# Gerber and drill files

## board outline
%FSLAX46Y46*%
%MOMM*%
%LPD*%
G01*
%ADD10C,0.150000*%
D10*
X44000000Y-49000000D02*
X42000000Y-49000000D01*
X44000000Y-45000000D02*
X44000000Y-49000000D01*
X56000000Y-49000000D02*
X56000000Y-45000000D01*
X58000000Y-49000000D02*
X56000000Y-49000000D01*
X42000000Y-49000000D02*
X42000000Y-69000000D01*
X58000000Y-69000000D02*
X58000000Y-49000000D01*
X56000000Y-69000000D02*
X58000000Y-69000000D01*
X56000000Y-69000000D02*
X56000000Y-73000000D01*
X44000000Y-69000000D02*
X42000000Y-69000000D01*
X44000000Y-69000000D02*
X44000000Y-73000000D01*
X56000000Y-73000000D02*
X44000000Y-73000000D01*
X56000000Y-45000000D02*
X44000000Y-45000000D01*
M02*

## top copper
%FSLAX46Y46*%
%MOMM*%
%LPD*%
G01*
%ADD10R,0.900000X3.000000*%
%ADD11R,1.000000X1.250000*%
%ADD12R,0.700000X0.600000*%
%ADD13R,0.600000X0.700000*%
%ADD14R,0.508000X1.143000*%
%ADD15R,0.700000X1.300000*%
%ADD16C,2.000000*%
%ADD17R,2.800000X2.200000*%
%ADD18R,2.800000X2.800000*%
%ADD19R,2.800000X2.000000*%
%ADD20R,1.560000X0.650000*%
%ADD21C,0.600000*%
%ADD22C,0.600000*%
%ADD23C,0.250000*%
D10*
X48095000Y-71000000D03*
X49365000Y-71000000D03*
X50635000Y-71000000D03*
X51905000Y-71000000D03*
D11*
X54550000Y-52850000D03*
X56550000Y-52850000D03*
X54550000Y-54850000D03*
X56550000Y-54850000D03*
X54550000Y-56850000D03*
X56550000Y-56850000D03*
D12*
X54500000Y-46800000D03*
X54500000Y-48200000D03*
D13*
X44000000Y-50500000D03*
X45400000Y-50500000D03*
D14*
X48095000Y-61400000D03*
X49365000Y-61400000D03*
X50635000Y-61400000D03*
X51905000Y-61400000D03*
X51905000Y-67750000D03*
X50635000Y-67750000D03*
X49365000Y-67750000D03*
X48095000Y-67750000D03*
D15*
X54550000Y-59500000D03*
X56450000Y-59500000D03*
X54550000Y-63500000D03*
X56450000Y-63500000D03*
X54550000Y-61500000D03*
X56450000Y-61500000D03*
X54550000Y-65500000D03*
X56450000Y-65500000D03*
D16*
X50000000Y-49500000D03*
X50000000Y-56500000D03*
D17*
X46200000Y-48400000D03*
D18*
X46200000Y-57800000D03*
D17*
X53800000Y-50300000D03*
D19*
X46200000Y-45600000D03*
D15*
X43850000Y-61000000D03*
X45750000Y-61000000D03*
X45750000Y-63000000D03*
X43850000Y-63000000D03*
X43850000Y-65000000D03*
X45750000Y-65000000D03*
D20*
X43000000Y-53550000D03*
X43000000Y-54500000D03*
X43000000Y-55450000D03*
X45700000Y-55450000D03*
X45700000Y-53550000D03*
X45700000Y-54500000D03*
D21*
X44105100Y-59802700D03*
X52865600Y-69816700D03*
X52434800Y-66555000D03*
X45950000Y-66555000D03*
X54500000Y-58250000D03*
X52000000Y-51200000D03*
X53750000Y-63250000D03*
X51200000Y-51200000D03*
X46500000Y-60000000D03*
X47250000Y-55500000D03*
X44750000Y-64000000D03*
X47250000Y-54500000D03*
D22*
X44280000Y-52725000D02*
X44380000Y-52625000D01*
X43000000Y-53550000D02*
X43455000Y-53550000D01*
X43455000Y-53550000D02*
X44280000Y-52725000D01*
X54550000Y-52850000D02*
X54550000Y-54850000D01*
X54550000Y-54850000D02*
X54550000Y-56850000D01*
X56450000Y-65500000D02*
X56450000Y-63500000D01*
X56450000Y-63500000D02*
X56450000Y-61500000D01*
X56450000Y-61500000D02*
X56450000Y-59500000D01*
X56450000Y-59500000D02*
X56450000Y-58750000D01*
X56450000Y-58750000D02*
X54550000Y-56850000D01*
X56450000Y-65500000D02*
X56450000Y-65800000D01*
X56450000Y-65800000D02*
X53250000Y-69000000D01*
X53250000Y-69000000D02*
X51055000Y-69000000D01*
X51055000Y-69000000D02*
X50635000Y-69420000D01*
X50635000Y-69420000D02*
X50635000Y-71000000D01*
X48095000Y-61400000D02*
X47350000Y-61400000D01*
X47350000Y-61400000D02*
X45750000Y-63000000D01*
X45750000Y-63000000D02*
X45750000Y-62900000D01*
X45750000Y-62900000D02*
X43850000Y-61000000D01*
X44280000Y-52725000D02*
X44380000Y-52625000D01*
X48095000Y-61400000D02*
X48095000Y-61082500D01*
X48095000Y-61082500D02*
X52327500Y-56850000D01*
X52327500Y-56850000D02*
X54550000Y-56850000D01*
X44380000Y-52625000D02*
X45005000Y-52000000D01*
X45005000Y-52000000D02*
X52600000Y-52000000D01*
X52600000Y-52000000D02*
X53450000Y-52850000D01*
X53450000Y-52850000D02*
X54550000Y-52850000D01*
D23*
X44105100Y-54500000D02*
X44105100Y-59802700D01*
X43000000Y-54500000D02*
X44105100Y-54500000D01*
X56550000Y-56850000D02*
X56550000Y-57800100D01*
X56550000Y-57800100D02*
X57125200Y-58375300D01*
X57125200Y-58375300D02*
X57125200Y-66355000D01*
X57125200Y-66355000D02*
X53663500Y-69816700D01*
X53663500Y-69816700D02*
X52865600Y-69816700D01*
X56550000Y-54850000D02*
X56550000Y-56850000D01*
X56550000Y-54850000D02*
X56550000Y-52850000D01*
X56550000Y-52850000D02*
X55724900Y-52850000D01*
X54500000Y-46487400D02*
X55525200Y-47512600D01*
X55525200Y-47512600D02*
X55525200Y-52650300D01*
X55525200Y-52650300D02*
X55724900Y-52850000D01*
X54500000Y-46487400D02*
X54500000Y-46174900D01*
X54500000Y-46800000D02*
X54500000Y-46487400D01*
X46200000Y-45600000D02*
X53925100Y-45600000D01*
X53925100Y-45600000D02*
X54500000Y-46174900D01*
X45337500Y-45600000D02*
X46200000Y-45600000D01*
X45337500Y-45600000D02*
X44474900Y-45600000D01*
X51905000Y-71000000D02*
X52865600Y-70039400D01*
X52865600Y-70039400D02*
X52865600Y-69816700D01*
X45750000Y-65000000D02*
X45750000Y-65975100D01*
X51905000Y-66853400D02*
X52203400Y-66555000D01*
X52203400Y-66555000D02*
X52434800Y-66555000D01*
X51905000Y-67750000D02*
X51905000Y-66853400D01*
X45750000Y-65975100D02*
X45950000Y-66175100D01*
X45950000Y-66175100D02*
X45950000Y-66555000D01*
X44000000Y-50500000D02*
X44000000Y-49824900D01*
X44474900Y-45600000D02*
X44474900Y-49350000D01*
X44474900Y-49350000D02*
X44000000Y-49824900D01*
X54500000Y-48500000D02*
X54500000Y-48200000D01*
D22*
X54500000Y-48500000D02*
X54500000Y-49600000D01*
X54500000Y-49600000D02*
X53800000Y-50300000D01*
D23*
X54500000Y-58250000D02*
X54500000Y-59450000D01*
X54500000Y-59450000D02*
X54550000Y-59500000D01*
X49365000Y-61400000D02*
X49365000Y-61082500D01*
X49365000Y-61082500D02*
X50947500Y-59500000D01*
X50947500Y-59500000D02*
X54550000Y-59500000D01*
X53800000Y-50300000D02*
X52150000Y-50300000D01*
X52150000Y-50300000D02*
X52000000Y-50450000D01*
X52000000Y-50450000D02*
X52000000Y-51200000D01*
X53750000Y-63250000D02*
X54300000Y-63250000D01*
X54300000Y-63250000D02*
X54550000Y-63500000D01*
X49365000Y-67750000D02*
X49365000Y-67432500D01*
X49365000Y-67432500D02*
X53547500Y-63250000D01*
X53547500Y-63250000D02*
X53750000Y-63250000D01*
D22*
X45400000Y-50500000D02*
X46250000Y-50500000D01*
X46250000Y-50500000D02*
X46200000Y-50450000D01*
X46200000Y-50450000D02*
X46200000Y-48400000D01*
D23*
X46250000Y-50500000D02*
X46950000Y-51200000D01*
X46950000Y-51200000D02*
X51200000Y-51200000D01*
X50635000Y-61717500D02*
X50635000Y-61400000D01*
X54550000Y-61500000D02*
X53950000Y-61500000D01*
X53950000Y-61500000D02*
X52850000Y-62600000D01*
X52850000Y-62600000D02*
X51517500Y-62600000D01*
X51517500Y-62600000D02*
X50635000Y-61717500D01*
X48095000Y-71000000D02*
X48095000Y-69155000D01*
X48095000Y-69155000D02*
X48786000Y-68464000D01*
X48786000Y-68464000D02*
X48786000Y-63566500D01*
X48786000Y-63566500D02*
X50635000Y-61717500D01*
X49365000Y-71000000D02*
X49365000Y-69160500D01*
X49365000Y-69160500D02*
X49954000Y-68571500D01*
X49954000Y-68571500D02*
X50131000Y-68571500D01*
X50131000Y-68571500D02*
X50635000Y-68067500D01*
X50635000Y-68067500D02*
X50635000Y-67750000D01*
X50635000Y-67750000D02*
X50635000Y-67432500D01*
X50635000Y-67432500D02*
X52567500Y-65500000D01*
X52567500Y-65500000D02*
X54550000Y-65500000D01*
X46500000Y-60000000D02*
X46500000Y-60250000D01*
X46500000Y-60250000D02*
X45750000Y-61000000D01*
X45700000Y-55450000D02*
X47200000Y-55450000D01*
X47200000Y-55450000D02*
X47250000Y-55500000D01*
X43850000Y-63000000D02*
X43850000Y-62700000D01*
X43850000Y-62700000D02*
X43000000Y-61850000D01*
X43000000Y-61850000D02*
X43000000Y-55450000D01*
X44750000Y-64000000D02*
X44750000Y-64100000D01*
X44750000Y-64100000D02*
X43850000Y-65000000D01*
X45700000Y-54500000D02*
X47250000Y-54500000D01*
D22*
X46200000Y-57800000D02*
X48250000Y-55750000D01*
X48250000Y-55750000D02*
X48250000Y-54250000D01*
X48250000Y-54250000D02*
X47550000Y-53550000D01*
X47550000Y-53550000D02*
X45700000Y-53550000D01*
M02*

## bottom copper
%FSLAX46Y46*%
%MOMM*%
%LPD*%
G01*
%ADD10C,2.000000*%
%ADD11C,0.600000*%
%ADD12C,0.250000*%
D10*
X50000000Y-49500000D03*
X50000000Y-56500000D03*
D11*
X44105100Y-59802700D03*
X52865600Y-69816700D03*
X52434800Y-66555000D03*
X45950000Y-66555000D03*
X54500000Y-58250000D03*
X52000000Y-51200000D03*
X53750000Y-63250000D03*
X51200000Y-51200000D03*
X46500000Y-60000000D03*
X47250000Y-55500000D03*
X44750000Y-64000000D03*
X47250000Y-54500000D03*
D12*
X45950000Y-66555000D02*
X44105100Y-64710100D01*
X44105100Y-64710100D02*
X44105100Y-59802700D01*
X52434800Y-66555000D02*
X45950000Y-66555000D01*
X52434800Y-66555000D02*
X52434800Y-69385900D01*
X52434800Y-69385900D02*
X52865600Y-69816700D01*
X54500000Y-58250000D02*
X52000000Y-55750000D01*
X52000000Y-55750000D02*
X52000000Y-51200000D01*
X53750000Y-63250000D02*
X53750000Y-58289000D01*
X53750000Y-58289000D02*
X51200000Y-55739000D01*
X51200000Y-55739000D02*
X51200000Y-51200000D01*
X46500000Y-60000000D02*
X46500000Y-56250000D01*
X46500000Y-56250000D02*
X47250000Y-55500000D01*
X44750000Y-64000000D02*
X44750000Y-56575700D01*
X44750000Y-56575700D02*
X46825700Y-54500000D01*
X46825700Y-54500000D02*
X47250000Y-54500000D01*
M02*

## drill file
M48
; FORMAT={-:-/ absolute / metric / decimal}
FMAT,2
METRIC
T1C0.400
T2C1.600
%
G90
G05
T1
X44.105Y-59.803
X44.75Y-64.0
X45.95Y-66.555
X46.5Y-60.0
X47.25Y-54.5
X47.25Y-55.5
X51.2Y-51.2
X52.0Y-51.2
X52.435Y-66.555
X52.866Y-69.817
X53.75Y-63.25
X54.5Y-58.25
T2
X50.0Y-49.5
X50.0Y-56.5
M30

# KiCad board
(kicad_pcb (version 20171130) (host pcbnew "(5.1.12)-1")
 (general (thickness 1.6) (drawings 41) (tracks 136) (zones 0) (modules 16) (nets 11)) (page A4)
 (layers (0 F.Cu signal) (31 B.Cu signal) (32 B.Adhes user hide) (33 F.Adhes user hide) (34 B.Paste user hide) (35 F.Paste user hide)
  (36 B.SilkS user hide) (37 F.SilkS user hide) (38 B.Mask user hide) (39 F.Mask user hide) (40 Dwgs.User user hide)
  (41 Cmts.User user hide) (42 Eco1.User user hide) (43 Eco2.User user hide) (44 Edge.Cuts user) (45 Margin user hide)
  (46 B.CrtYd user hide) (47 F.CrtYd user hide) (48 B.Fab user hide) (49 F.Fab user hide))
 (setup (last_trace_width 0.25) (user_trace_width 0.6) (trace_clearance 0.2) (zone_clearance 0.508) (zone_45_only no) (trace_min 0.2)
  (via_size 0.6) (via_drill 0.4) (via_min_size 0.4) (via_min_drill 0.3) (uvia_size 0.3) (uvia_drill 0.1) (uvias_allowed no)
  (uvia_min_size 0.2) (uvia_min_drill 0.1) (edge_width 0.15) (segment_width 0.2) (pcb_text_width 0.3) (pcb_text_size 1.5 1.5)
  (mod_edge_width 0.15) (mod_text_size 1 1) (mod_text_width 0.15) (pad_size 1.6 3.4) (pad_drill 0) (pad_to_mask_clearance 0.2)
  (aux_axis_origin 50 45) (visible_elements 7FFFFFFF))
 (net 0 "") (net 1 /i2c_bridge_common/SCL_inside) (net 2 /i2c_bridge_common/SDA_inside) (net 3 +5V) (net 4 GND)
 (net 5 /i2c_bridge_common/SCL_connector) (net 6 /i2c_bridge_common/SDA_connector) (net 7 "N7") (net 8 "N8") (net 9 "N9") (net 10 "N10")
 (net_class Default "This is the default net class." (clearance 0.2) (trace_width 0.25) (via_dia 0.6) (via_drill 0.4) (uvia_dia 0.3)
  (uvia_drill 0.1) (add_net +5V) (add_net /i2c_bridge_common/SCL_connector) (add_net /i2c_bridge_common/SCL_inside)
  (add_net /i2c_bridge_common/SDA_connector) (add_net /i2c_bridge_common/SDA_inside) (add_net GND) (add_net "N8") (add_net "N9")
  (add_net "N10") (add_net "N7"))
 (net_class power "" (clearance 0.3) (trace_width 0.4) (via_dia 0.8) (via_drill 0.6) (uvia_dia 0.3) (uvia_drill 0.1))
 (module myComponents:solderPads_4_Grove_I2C (layer F.Cu) (at 50 71)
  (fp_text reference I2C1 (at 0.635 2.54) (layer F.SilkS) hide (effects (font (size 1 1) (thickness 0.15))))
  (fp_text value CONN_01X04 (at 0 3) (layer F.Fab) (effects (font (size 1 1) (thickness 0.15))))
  (pad 1 smd rect (at -1.905 0) (size 0.9 3) (layers F.Cu F.Paste F.Mask) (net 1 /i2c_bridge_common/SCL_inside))
  (pad 2 smd rect (at -0.635 0) (size 0.9 3) (layers F.Cu F.Paste F.Mask) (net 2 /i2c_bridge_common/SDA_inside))
  (pad 3 smd rect (at 0.635 0) (size 0.9 3) (layers F.Cu F.Paste F.Mask) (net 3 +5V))
  (pad 4 smd rect (at 1.905 0) (size 0.9 3) (layers F.Cu F.Paste F.Mask) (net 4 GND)))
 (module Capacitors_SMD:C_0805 (layer F.Cu) (at 55.55 52.85)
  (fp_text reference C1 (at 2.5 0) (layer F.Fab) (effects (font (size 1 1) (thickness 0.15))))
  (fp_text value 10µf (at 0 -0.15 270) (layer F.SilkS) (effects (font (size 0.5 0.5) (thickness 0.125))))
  (pad 1 smd rect (at -1 0) (size 1 1.25) (layers F.Cu F.Paste F.Mask) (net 3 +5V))
  (pad 2 smd rect (at 1 0) (size 1 1.25) (layers F.Cu F.Paste F.Mask) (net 4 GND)))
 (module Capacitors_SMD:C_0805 (layer F.Cu) (at 55.55 54.85)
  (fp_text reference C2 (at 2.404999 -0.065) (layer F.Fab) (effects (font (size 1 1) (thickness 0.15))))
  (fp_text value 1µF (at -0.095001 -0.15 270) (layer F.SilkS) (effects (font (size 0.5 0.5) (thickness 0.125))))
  (pad 1 smd rect (at -1 0) (size 1 1.25) (layers F.Cu F.Paste F.Mask) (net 3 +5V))
  (pad 2 smd rect (at 1 0) (size 1 1.25) (layers F.Cu F.Paste F.Mask) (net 4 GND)))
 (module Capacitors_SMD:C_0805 (layer F.Cu) (at 55.55 56.85)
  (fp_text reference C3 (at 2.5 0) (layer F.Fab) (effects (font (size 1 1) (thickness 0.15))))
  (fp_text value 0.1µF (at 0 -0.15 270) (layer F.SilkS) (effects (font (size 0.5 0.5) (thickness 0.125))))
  (pad 1 smd rect (at -1 0) (size 1 1.25) (layers F.Cu F.Paste F.Mask) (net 3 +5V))
  (pad 2 smd rect (at 1 0) (size 1 1.25) (layers F.Cu F.Paste F.Mask) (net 4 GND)))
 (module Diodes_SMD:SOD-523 (layer F.Cu) (at 54.5 47.5 90)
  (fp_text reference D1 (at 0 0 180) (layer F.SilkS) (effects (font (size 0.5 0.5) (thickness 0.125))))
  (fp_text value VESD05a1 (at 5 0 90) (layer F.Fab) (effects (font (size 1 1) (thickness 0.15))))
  (pad 2 smd rect (at 0.7 0 270) (size 0.6 0.7) (layers F.Cu F.Paste F.Mask) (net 4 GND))
  (pad 1 smd rect (at -0.7 0 270) (size 0.6 0.7) (layers F.Cu F.Paste F.Mask) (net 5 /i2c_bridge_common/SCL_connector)))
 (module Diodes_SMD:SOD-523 (layer F.Cu) (at 44.7 50.5 180)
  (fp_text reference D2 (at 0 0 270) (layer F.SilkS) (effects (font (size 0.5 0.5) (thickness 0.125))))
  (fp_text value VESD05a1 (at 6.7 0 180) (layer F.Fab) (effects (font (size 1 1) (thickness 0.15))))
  (pad 2 smd rect (at 0.7 0) (size 0.6 0.7) (layers F.Cu F.Paste F.Mask) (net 4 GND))
  (pad 1 smd rect (at -0.7 0) (size 0.6 0.7) (layers F.Cu F.Paste F.Mask) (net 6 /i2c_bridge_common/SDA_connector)))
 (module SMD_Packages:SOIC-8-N (layer F.Cu) (at 50 64.575)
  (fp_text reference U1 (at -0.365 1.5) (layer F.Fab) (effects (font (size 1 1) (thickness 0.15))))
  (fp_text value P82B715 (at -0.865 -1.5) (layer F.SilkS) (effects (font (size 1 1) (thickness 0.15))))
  (pad 8 smd rect (at -1.905 -3.175) (size 0.508 1.143) (layers F.Cu F.Paste F.Mask) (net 3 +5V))
  (pad 7 smd rect (at -0.635 -3.175) (size 0.508 1.143) (layers F.Cu F.Paste F.Mask) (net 5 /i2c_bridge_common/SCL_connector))
  (pad 6 smd rect (at 0.635 -3.175) (size 0.508 1.143) (layers F.Cu F.Paste F.Mask) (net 1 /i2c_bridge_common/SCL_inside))
  (pad 5 smd rect (at 1.905 -3.175) (size 0.508 1.143) (layers F.Cu F.Paste F.Mask))
  (pad 4 smd rect (at 1.905 3.175) (size 0.508 1.143) (layers F.Cu F.Paste F.Mask) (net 4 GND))
  (pad 3 smd rect (at 0.635 3.175) (size 0.508 1.143) (layers F.Cu F.Paste F.Mask) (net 2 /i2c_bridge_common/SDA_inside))
  (pad 2 smd rect (at -0.635 3.175) (size 0.508 1.143) (layers F.Cu F.Paste F.Mask) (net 6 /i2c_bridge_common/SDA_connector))
  (pad 1 smd rect (at -1.905 3.175) (size 0.508 1.143) (layers F.Cu F.Paste F.Mask)))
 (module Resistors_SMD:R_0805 (layer F.Cu) (at 55.5 59.5)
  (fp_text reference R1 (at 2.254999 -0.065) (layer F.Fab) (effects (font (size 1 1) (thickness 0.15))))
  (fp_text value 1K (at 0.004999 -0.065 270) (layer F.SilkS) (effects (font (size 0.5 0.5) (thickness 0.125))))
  (pad 1 smd rect (at -0.95 0) (size 0.7 1.3) (layers F.Cu F.Paste F.Mask) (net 5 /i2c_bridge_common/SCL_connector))
  (pad 2 smd rect (at 0.95 0) (size 0.7 1.3) (layers F.Cu F.Paste F.Mask) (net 3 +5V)))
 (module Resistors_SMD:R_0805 (layer F.Cu) (at 55.5 63.5)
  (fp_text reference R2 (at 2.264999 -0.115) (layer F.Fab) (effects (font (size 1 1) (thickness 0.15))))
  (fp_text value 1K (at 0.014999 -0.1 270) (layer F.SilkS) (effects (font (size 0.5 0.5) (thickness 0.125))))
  (pad 1 smd rect (at -0.95 0) (size 0.7 1.3) (layers F.Cu F.Paste F.Mask) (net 6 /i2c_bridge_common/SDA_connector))
  (pad 2 smd rect (at 0.95 0) (size 0.7 1.3) (layers F.Cu F.Paste F.Mask) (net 3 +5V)))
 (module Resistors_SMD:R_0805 (layer F.Cu) (at 55.5 61.5)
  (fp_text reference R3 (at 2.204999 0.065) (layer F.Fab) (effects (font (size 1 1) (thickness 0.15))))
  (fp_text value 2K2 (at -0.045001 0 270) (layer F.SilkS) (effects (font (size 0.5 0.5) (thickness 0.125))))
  (pad 1 smd rect (at -0.95 0) (size 0.7 1.3) (layers F.Cu F.Paste F.Mask) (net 1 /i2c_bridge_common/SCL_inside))
  (pad 2 smd rect (at 0.95 0) (size 0.7 1.3) (layers F.Cu F.Paste F.Mask) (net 3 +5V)))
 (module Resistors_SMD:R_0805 (layer F.Cu) (at 55.5 65.5)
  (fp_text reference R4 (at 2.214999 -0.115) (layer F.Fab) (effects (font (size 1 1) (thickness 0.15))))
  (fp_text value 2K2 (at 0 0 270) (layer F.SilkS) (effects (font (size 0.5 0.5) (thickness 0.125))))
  (pad 1 smd rect (at -0.95 0) (size 0.7 1.3) (layers F.Cu F.Paste F.Mask) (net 2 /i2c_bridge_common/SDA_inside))
  (pad 2 smd rect (at 0.95 0) (size 0.7 1.3) (layers F.Cu F.Paste F.Mask) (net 3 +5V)))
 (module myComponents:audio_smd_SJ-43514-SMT (layer F.Cu) (at 50 45 270)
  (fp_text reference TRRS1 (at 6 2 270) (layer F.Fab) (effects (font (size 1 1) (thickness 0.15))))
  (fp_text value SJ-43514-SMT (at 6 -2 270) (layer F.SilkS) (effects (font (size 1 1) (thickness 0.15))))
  (pad "" thru_hole circle (at 4.5 0 270) (size 2 2) (drill 1.6) (layers *.Cu *.Mask F.SilkS))
  (pad "" thru_hole circle (at 11.5 0 270) (size 2 2) (drill 1.6) (layers *.Cu *.Mask F.SilkS))
  (pad 4 smd rect (at 3.4 3.8 270) (size 2.2 2.8) (layers F.Cu F.Paste F.Mask) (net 6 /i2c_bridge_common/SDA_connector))
  (pad 2 smd rect (at 12.8 3.8 270) (size 2.8 2.8) (layers F.Cu F.Paste F.Mask) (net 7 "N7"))
  (pad 3 smd rect (at 5.3 -3.8 270) (size 2.2 2.8) (layers F.Cu F.Paste F.Mask) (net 5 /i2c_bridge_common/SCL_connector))
  (pad 1 smd rect (at 0.6 3.8 270) (size 2 2.8) (layers F.Cu F.Paste F.Mask) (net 4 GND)))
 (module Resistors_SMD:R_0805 (layer F.Cu) (at 44.8 61)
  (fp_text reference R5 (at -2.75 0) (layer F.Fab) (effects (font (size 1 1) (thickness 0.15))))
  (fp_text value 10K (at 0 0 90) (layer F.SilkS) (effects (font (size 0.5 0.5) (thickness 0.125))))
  (pad 1 smd rect (at -0.95 0) (size 0.7 1.3) (layers F.Cu F.Paste F.Mask) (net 3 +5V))
  (pad 2 smd rect (at 0.95 0) (size 0.7 1.3) (layers F.Cu F.Paste F.Mask) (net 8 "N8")))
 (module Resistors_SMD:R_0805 (layer F.Cu) (at 44.8 63 180)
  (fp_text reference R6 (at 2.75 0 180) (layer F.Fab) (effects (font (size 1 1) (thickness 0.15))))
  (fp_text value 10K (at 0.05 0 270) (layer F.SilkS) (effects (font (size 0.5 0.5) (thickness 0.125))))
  (pad 1 smd rect (at -0.95 0 180) (size 0.7 1.3) (layers F.Cu F.Paste F.Mask) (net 3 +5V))
  (pad 2 smd rect (at 0.95 0 180) (size 0.7 1.3) (layers F.Cu F.Paste F.Mask) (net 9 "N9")))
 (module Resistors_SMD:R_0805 (layer F.Cu) (at 44.8 65)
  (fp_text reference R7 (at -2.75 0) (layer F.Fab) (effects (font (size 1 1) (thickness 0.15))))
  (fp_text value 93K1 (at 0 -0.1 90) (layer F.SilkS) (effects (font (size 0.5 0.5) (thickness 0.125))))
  (pad 1 smd rect (at -0.95 0) (size 0.7 1.3) (layers F.Cu F.Paste F.Mask) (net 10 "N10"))
  (pad 2 smd rect (at 0.95 0) (size 0.7 1.3) (layers F.Cu F.Paste F.Mask) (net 4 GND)))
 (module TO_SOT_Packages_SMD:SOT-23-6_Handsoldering (layer F.Cu) (at 44.35 54.5)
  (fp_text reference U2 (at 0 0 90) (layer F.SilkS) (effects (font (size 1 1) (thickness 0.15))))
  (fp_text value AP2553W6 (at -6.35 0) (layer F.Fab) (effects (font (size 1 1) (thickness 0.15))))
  (pad 1 smd rect (at -1.35 -0.95) (size 1.56 0.65) (layers F.Cu F.Paste F.Mask) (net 3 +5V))
  (pad 2 smd rect (at -1.35 0) (size 1.56 0.65) (layers F.Cu F.Paste F.Mask) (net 4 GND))
  (pad 3 smd rect (at -1.35 0.95) (size 1.56 0.65) (layers F.Cu F.Paste F.Mask) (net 9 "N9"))
  (pad 4 smd rect (at 1.35 0.95) (size 1.56 0.65) (layers F.Cu F.Paste F.Mask) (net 8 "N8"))
  (pad 6 smd rect (at 1.35 -0.95) (size 1.56 0.65) (layers F.Cu F.Paste F.Mask) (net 7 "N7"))
  (pad 5 smd rect (at 1.35 0) (size 1.56 0.65) (layers F.Cu F.Paste F.Mask) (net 10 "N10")))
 (gr_line (start 44 49) (end 42 49) (layer Edge.Cuts) (width 0.15))
 (gr_line (start 44 45) (end 44 49) (layer Edge.Cuts) (width 0.15))
 (gr_line (start 56 49) (end 56 45) (layer Edge.Cuts) (width 0.15))
 (gr_line (start 58 49) (end 56 49) (layer Edge.Cuts) (width 0.15))
 (gr_line (start 42 49) (end 42 69) (layer Edge.Cuts) (width 0.15))
 (gr_line (start 58 69) (end 58 49) (layer Edge.Cuts) (width 0.15))
 (gr_line (start 56 69) (end 58 69) (layer Edge.Cuts) (width 0.15))
 (gr_line (start 56 69) (end 56 73) (layer Edge.Cuts) (width 0.15))
 (gr_line (start 44 69) (end 42 69) (layer Edge.Cuts) (width 0.15))
 (gr_line (start 44 69) (end 44 73) (layer Edge.Cuts) (width 0.15))
 (gr_line (start 56 73) (end 44 73) (layer Edge.Cuts) (width 0.15))
 (gr_line (start 56 45) (end 44 45) (layer Edge.Cuts) (width 0.15))
 (segment (start 44.28 52.725) (end 44.38 52.625) (width 0.6) (layer F.Cu) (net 3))
 (segment (start 43 53.55) (end 43.455 53.55) (width 0.6) (layer F.Cu) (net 3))
 (segment (start 43.455 53.55) (end 44.28 52.725) (width 0.6) (layer F.Cu) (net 3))
 (segment (start 54.55 52.85) (end 54.55 54.85) (width 0.6) (layer F.Cu) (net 3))
 (segment (start 54.55 54.85) (end 54.55 56.85) (width 0.6) (layer F.Cu) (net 3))
 (segment (start 56.45 65.5) (end 56.45 63.5) (width 0.6) (layer F.Cu) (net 3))
 (segment (start 56.45 63.5) (end 56.45 61.5) (width 0.6) (layer F.Cu) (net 3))
 (segment (start 56.45 61.5) (end 56.45 59.5) (width 0.6) (layer F.Cu) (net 3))
 (segment (start 56.45 59.5) (end 56.45 58.75) (width 0.6) (layer F.Cu) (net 3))
 (segment (start 56.45 58.75) (end 54.55 56.85) (width 0.6) (layer F.Cu) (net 3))
 (segment (start 56.45 65.5) (end 56.45 65.8) (width 0.6) (layer F.Cu) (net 3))
 (segment (start 56.45 65.8) (end 53.25 69) (width 0.6) (layer F.Cu) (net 3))
 (segment (start 53.25 69) (end 51.055 69) (width 0.6) (layer F.Cu) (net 3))
 (segment (start 51.055 69) (end 50.635 69.42) (width 0.6) (layer F.Cu) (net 3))
 (segment (start 50.635 69.42) (end 50.635 71) (width 0.6) (layer F.Cu) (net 3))
 (segment (start 48.095 61.4) (end 47.35 61.4) (width 0.6) (layer F.Cu) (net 3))
 (segment (start 47.35 61.4) (end 45.75 63) (width 0.6) (layer F.Cu) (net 3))
 (segment (start 45.75 63) (end 45.75 62.9) (width 0.6) (layer F.Cu) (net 3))
 (segment (start 45.75 62.9) (end 43.85 61) (width 0.6) (layer F.Cu) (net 3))
 (segment (start 44.28 52.725) (end 44.38 52.625) (width 0.6) (layer F.Cu) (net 3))
 (segment (start 48.095 61.4) (end 48.095 61.0825) (width 0.6) (layer F.Cu) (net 3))
 (segment (start 48.095 61.0825) (end 52.3275 56.85) (width 0.6) (layer F.Cu) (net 3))
 (segment (start 52.3275 56.85) (end 54.55 56.85) (width 0.6) (layer F.Cu) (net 3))
 (segment (start 44.38 52.625) (end 45.005 52) (width 0.6) (layer F.Cu) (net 3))
 (segment (start 45.005 52) (end 52.6 52) (width 0.6) (layer F.Cu) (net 3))
 (segment (start 52.6 52) (end 53.45 52.85) (width 0.6) (layer F.Cu) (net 3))
 (segment (start 53.45 52.85) (end 54.55 52.85) (width 0.6) (layer F.Cu) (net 3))
 (segment (start 44.1051 54.5) (end 44.1051 59.8027) (width 0.25) (layer F.Cu) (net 4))
 (segment (start 45.95 66.555) (end 44.1051 64.7101) (width 0.25) (layer B.Cu) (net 4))
 (segment (start 44.1051 64.7101) (end 44.1051 59.8027) (width 0.25) (layer B.Cu) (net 4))
 (segment (start 43 54.5) (end 44.1051 54.5) (width 0.25) (layer F.Cu) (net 4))
 (segment (start 52.4348 66.555) (end 45.95 66.555) (width 0.25) (layer B.Cu) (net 4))
 (segment (start 56.55 56.85) (end 56.55 57.8001) (width 0.25) (layer F.Cu) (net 4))
 (segment (start 56.55 57.8001) (end 57.1252 58.3753) (width 0.25) (layer F.Cu) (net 4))
 (segment (start 57.1252 58.3753) (end 57.1252 66.355) (width 0.25) (layer F.Cu) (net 4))
 (segment (start 57.1252 66.355) (end 53.6635 69.8167) (width 0.25) (layer F.Cu) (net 4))
 (segment (start 53.6635 69.8167) (end 52.8656 69.8167) (width 0.25) (layer F.Cu) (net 4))
 (segment (start 56.55 54.85) (end 56.55 56.85) (width 0.25) (layer F.Cu) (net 4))
 (segment (start 56.55 54.85) (end 56.55 52.85) (width 0.25) (layer F.Cu) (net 4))
 (segment (start 56.55 52.85) (end 55.7249 52.85) (width 0.25) (layer F.Cu) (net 4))
 (segment (start 54.5 46.4874) (end 55.5252 47.5126) (width 0.25) (layer F.Cu) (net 4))
 (segment (start 55.5252 47.5126) (end 55.5252 52.6503) (width 0.25) (layer F.Cu) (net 4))
 (segment (start 55.5252 52.6503) (end 55.7249 52.85) (width 0.25) (layer F.Cu) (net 4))
 (segment (start 54.5 46.4874) (end 54.5 46.1749) (width 0.25) (layer F.Cu) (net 4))
 (segment (start 54.5 46.8) (end 54.5 46.4874) (width 0.25) (layer F.Cu) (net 4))
 (segment (start 46.2 45.6) (end 53.9251 45.6) (width 0.25) (layer F.Cu) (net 4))
 (segment (start 53.9251 45.6) (end 54.5 46.1749) (width 0.25) (layer F.Cu) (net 4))
 (segment (start 45.3375 45.6) (end 46.2 45.6) (width 0.25) (layer F.Cu) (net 4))
 (segment (start 45.3375 45.6) (end 44.4749 45.6) (width 0.25) (layer F.Cu) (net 4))
 (segment (start 52.4348 66.555) (end 52.4348 69.3859) (width 0.25) (layer B.Cu) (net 4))
 (segment (start 52.4348 69.3859) (end 52.8656 69.8167) (width 0.25) (layer B.Cu) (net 4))
 (segment (start 51.905 71) (end 52.8656 70.0394) (width 0.25) (layer F.Cu) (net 4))
 (segment (start 52.8656 70.0394) (end 52.8656 69.8167) (width 0.25) (layer F.Cu) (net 4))
 (segment (start 45.75 65) (end 45.75 65.9751) (width 0.25) (layer F.Cu) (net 4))
 (segment (start 51.905 66.8534) (end 52.2034 66.555) (width 0.25) (layer F.Cu) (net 4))
 (segment (start 52.2034 66.555) (end 52.4348 66.555) (width 0.25) (layer F.Cu) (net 4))
 (segment (start 51.905 67.75) (end 51.905 66.8534) (width 0.25) (layer F.Cu) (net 4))
 (segment (start 45.75 65.9751) (end 45.95 66.1751) (width 0.25) (layer F.Cu) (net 4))
 (segment (start 45.95 66.1751) (end 45.95 66.555) (width 0.25) (layer F.Cu) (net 4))
 (segment (start 44 50.5) (end 44 49.8249) (width 0.25) (layer F.Cu) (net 4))
 (segment (start 44.4749 45.6) (end 44.4749 49.35) (width 0.25) (layer F.Cu) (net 4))
 (segment (start 44.4749 49.35) (end 44 49.8249) (width 0.25) (layer F.Cu) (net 4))
 (via (at 44.1051 59.8027) (size 0.6) (layers F.Cu B.Cu) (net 4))
 (via (at 52.8656 69.8167) (size 0.6) (layers F.Cu B.Cu) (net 4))
 (via (at 52.4348 66.555) (size 0.6) (layers F.Cu B.Cu) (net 4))
 (via (at 45.95 66.555) (size 0.6) (layers F.Cu B.Cu) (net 4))
 (segment (start 54.5 48.5) (end 54.5 48.2) (width 0.25) (layer F.Cu) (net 5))
 (segment (start 54.5 48.5) (end 54.5 49.6) (width 0.6) (layer F.Cu) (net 5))
 (segment (start 54.5 49.6) (end 53.8 50.3) (width 0.6) (layer F.Cu) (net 5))
 (segment (start 54.5 58.25) (end 54.5 59.45) (width 0.25) (layer F.Cu) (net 5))
 (segment (start 54.5 59.45) (end 54.55 59.5) (width 0.25) (layer F.Cu) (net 5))
 (segment (start 49.365 61.4) (end 49.365 61.0825) (width 0.25) (layer F.Cu) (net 5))
 (segment (start 49.365 61.0825) (end 50.9475 59.5) (width 0.25) (layer F.Cu) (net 5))
 (segment (start 50.9475 59.5) (end 54.55 59.5) (width 0.25) (layer F.Cu) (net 5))
 (segment (start 53.8 50.3) (end 52.15 50.3) (width 0.25) (layer F.Cu) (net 5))
 (segment (start 52.15 50.3) (end 52 50.45) (width 0.25) (layer F.Cu) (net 5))
 (segment (start 52 50.45) (end 52 51.2) (width 0.25) (layer F.Cu) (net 5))
 (segment (start 54.5 58.25) (end 52 55.75) (width 0.25) (layer B.Cu) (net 5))
 (segment (start 52 55.75) (end 52 51.2) (width 0.25) (layer B.Cu) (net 5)) (via (at 54.5 58.25) (size 0.6) (layers F.Cu B.Cu) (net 5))
 (via (at 52 51.2) (size 0.6) (layers F.Cu B.Cu) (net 5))
 (segment (start 53.75 63.25) (end 54.3 63.25) (width 0.25) (layer F.Cu) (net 6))
 (segment (start 54.3 63.25) (end 54.55 63.5) (width 0.25) (layer F.Cu) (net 6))
 (segment (start 49.365 67.75) (end 49.365 67.4325) (width 0.25) (layer F.Cu) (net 6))
 (segment (start 49.365 67.4325) (end 53.5475 63.25) (width 0.25) (layer F.Cu) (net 6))
 (segment (start 53.5475 63.25) (end 53.75 63.25) (width 0.25) (layer F.Cu) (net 6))
 (segment (start 45.4 50.5) (end 46.25 50.5) (width 0.6) (layer F.Cu) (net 6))
 (segment (start 46.25 50.5) (end 46.2 50.45) (width 0.6) (layer F.Cu) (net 6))
 (segment (start 46.2 50.45) (end 46.2 48.4) (width 0.6) (layer F.Cu) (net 6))
 (segment (start 53.75 63.25) (end 53.75 58.289) (width 0.25) (layer B.Cu) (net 6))
 (segment (start 53.75 58.289) (end 51.2 55.739) (width 0.25) (layer B.Cu) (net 6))
 (segment (start 51.2 55.739) (end 51.2 51.2) (width 0.25) (layer B.Cu) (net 6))
 (segment (start 46.25 50.5) (end 46.95 51.2) (width 0.25) (layer F.Cu) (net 6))
 (segment (start 46.95 51.2) (end 51.2 51.2) (width 0.25) (layer F.Cu) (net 6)) (via (at 53.75 63.25) (size 0.6) (layers F.Cu B.Cu) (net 6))
 (via (at 51.2 51.2) (size 0.6) (layers F.Cu B.Cu) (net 6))
 (segment (start 50.635 61.7175) (end 50.635 61.4) (width 0.25) (layer F.Cu) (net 1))
 (segment (start 54.55 61.5) (end 53.95 61.5) (width 0.25) (layer F.Cu) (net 1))
 (segment (start 53.95 61.5) (end 52.85 62.6) (width 0.25) (layer F.Cu) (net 1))
 (segment (start 52.85 62.6) (end 51.5175 62.6) (width 0.25) (layer F.Cu) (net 1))
 (segment (start 51.5175 62.6) (end 50.635 61.7175) (width 0.25) (layer F.Cu) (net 1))
 (segment (start 48.095 71) (end 48.095 69.155) (width 0.25) (layer F.Cu) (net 1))
 (segment (start 48.095 69.155) (end 48.786 68.464) (width 0.25) (layer F.Cu) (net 1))
 (segment (start 48.786 68.464) (end 48.786 63.5665) (width 0.25) (layer F.Cu) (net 1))
 (segment (start 48.786 63.5665) (end 50.635 61.7175) (width 0.25) (layer F.Cu) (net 1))
 (segment (start 49.365 71) (end 49.365 69.1605) (width 0.25) (layer F.Cu) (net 2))
 (segment (start 49.365 69.1605) (end 49.954 68.5715) (width 0.25) (layer F.Cu) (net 2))
 (segment (start 49.954 68.5715) (end 50.131 68.5715) (width 0.25) (layer F.Cu) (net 2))
 (segment (start 50.131 68.5715) (end 50.635 68.0675) (width 0.25) (layer F.Cu) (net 2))
 (segment (start 50.635 68.0675) (end 50.635 67.75) (width 0.25) (layer F.Cu) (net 2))
 (segment (start 50.635 67.75) (end 50.635 67.4325) (width 0.25) (layer F.Cu) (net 2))
 (segment (start 50.635 67.4325) (end 52.5675 65.5) (width 0.25) (layer F.Cu) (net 2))
 (segment (start 52.5675 65.5) (end 54.55 65.5) (width 0.25) (layer F.Cu) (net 2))
 (segment (start 46.5 60) (end 46.5 60.25) (width 0.25) (layer F.Cu) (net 8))
 (segment (start 46.5 60.25) (end 45.75 61) (width 0.25) (layer F.Cu) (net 8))
 (segment (start 46.5 60) (end 46.5 56.25) (width 0.25) (layer B.Cu) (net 8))
 (segment (start 46.5 56.25) (end 47.25 55.5) (width 0.25) (layer B.Cu) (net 8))
 (segment (start 45.7 55.45) (end 47.2 55.45) (width 0.25) (layer F.Cu) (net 8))
 (segment (start 47.2 55.45) (end 47.25 55.5) (width 0.25) (layer F.Cu) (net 8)) (via (at 46.5 60) (size 0.6) (layers F.Cu B.Cu) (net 8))
 (via (at 47.25 55.5) (size 0.6) (layers F.Cu B.Cu) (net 8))
 (segment (start 43.85 63) (end 43.85 62.7) (width 0.25) (layer F.Cu) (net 9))
 (segment (start 43.85 62.7) (end 43 61.85) (width 0.25) (layer F.Cu) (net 9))
 (segment (start 43 61.85) (end 43 55.45) (width 0.25) (layer F.Cu) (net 9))
 (segment (start 44.75 64) (end 44.75 64.1) (width 0.25) (layer F.Cu) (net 10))
 (segment (start 44.75 64.1) (end 43.85 65) (width 0.25) (layer F.Cu) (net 10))
 (segment (start 45.7 54.5) (end 47.25 54.5) (width 0.25) (layer F.Cu) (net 10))
 (segment (start 44.75 64) (end 44.75 56.5757) (width 0.25) (layer B.Cu) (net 10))
 (segment (start 44.75 56.5757) (end 46.8257 54.5) (width 0.25) (layer B.Cu) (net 10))
 (segment (start 46.8257 54.5) (end 47.25 54.5) (width 0.25) (layer B.Cu) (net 10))
 (via (at 44.75 64) (size 0.6) (layers F.Cu B.Cu) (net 10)) (via (at 47.25 54.5) (size 0.6) (layers F.Cu B.Cu) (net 10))
 (segment (start 46.2 57.8) (end 48.25 55.75) (width 0.6) (layer F.Cu) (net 7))
 (segment (start 48.25 55.75) (end 48.25 54.25) (width 0.6) (layer F.Cu) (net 7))
 (segment (start 48.25 54.25) (end 47.55 53.55) (width 0.6) (layer F.Cu) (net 7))
 (segment (start 47.55 53.55) (end 45.7 53.55) (width 0.6) (layer F.Cu) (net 7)))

